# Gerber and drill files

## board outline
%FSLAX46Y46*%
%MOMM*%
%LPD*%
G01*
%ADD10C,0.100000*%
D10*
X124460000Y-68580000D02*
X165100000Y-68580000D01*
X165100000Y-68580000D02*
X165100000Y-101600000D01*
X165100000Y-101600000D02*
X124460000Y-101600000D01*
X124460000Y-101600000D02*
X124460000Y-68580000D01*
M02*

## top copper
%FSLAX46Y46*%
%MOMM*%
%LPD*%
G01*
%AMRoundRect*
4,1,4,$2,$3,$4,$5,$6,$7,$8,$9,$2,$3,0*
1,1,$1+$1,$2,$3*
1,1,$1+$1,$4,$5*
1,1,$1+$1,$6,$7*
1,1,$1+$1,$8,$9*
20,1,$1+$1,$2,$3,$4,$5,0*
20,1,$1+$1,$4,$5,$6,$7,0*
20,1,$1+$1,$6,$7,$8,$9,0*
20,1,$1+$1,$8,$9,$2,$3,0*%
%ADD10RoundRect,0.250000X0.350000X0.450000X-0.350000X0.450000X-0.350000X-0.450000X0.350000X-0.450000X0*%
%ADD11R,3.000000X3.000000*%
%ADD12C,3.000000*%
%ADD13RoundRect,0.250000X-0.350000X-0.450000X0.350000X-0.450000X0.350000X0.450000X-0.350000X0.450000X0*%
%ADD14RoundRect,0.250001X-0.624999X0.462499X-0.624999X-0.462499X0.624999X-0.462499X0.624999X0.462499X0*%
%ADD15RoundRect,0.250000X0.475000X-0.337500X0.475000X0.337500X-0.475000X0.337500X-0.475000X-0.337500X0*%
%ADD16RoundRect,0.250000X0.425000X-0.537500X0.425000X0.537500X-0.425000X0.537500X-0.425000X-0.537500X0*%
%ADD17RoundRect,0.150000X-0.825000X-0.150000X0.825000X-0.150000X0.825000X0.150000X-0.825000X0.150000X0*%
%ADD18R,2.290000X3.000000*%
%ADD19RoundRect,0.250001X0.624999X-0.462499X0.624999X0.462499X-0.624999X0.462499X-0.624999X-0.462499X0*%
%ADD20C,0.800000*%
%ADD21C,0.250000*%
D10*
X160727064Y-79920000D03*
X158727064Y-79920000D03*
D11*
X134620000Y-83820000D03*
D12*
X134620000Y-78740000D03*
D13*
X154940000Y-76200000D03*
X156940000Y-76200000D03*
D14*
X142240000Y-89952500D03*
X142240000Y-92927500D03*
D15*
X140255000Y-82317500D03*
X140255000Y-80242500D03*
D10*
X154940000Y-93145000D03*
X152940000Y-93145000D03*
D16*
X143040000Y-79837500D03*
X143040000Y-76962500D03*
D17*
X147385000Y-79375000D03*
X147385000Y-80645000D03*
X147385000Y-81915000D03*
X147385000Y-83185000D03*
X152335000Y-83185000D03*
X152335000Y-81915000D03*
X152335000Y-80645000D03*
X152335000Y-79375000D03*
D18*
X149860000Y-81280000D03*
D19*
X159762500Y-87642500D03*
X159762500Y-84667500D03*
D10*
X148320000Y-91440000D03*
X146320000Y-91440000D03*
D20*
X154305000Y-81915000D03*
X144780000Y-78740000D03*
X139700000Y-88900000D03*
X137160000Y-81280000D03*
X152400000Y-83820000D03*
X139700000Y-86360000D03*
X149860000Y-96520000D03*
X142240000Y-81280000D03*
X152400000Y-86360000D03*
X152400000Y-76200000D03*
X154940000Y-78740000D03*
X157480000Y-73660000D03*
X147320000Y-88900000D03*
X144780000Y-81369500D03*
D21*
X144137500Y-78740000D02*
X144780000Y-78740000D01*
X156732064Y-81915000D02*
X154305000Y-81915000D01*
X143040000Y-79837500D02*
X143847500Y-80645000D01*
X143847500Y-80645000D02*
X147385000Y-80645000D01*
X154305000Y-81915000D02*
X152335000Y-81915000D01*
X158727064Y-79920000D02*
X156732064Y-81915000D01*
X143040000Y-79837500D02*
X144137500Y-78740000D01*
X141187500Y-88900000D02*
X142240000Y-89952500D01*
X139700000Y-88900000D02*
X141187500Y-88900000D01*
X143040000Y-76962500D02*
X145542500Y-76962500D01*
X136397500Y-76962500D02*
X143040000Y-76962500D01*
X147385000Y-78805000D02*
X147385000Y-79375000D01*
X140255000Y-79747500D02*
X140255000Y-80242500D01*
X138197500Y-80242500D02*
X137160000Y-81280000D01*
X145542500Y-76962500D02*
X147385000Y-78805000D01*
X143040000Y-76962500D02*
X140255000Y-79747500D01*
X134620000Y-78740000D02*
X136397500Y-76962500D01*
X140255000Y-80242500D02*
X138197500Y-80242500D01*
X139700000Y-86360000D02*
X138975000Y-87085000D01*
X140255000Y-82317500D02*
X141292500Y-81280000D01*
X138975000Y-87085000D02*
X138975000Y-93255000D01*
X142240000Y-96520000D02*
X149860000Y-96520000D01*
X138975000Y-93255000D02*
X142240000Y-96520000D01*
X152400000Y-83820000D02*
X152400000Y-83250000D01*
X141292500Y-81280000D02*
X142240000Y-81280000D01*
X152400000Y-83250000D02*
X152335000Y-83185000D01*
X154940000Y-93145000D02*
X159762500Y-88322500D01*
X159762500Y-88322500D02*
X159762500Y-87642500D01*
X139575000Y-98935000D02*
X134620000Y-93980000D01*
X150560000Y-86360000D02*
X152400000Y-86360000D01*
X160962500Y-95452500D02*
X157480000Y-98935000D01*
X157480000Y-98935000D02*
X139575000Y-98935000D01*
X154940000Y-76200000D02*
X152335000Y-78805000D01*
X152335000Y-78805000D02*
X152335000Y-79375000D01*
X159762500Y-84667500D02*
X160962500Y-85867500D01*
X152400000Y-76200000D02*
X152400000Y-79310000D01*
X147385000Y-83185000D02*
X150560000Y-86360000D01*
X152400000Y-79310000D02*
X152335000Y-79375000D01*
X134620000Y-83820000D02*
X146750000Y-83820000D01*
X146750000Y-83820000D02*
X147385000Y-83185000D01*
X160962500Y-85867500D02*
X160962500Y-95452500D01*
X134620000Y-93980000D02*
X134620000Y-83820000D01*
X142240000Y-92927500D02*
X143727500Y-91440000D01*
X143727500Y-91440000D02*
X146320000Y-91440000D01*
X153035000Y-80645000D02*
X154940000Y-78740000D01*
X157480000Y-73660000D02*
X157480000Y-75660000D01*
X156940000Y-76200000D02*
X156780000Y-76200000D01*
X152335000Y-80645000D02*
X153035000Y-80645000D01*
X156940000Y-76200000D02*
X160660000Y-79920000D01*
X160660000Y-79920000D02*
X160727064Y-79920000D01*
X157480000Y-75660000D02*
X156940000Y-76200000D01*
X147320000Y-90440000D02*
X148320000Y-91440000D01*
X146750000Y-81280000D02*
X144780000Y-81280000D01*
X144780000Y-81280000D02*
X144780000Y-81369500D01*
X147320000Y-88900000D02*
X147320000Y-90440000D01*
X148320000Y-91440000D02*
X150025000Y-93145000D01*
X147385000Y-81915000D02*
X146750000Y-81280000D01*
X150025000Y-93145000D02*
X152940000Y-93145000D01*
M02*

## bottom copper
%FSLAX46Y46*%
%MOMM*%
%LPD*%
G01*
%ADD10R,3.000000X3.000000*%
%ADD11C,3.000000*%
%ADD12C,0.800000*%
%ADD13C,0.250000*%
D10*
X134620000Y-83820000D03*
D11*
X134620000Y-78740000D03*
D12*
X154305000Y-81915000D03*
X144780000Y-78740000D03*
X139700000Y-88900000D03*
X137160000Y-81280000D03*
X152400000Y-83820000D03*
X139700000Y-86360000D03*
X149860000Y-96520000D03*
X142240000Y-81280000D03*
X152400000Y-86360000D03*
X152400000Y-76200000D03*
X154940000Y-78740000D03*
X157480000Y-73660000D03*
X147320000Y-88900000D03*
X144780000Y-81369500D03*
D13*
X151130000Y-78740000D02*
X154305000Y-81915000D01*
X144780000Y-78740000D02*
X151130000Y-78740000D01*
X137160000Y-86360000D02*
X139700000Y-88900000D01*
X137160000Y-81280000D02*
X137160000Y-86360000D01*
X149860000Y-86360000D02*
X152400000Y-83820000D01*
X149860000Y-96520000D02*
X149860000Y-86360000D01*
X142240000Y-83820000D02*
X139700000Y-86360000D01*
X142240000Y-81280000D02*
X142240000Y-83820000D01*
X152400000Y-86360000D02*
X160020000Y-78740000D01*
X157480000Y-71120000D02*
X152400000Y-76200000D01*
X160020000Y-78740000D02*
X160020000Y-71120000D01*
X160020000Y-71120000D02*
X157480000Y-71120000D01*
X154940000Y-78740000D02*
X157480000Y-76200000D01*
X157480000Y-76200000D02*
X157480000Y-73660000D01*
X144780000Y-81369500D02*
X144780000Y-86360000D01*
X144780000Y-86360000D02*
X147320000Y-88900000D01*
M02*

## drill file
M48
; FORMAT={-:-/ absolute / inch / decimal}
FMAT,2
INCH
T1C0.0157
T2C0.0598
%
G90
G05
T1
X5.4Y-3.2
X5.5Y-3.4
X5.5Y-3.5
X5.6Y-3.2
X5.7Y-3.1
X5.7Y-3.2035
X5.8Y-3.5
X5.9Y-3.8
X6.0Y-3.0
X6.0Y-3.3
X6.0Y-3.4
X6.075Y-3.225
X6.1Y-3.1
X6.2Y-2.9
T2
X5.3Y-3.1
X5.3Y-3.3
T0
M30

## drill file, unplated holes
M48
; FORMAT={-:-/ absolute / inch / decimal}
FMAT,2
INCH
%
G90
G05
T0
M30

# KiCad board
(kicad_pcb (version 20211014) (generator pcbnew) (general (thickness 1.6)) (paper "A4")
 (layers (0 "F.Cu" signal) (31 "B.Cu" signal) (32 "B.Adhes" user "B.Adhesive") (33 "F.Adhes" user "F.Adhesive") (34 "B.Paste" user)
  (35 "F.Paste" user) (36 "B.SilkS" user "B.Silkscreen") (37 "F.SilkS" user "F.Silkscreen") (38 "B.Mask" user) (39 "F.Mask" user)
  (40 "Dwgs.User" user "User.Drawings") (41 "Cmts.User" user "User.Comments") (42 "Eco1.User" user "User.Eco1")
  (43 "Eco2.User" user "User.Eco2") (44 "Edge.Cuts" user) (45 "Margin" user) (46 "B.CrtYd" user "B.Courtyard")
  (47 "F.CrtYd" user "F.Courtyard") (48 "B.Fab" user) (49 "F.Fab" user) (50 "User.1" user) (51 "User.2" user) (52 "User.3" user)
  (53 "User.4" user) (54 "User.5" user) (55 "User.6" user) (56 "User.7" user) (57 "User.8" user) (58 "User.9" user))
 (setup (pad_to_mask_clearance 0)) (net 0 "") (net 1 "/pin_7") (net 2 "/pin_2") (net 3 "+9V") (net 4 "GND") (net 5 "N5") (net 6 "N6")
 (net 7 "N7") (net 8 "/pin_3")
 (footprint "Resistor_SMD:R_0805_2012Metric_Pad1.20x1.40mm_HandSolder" (layer "F.Cu") (at 159.727064 79.92 180)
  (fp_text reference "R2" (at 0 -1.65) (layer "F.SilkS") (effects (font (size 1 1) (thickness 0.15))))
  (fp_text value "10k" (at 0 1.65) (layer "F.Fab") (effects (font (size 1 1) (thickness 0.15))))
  (pad "1" smd roundrect (at -1 0 180) (size 1.2 1.4) (layers "F.Cu" "F.Paste" "F.Mask") (roundrect_rratio 0.2083333333) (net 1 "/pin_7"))
  (pad "2" smd roundrect (at 1 0 180) (size 1.2 1.4) (layers "F.Cu" "F.Paste" "F.Mask") (roundrect_rratio 0.2083333333) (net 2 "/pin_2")))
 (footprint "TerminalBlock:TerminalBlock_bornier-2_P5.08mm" (layer "F.Cu") (at 134.62 83.82 90)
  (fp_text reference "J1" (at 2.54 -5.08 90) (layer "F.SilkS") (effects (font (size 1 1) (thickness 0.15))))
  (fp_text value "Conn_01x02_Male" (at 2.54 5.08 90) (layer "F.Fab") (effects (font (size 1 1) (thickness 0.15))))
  (pad "1" thru_hole rect (at 0 0 90) (size 3 3) (drill 1.52) (layers *.Cu *.Mask) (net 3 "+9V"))
  (pad "2" thru_hole circle (at 5.08 0 90) (size 3 3) (drill 1.52) (layers *.Cu *.Mask) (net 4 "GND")))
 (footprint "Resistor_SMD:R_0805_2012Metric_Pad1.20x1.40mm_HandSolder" (layer "F.Cu") (at 155.94 76.2)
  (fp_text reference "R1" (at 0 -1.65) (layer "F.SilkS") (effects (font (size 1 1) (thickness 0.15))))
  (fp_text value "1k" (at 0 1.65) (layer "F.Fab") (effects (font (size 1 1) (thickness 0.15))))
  (pad "1" smd roundrect (at -1 0) (size 1.2 1.4) (layers "F.Cu" "F.Paste" "F.Mask") (roundrect_rratio 0.2083333333) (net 3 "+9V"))
  (pad "2" smd roundrect (at 1 0) (size 1.2 1.4) (layers "F.Cu" "F.Paste" "F.Mask") (roundrect_rratio 0.2083333333) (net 1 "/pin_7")))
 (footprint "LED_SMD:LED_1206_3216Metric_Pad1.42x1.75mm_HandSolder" (layer "F.Cu") (at 142.24 91.44 -90)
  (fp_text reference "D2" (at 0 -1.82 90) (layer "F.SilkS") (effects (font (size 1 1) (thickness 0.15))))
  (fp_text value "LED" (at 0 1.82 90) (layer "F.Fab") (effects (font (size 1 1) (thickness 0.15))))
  (pad "1" smd roundrect (at -1.4875 0 270) (size 1.425 1.75) (layers "F.Cu" "F.Paste" "F.Mask") (roundrect_rratio 0.1754392982)
   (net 4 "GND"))
  (pad "2" smd roundrect (at 1.4875 0 270) (size 1.425 1.75) (layers "F.Cu" "F.Paste" "F.Mask") (roundrect_rratio 0.1754392982) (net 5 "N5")))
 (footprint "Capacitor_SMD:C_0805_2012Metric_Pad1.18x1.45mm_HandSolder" (layer "F.Cu") (at 140.255 81.28 90)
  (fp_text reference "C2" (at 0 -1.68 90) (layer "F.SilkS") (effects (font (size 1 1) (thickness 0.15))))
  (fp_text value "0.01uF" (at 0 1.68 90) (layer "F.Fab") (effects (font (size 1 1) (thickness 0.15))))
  (pad "1" smd roundrect (at -1.0375 0 90) (size 1.175 1.45) (layers "F.Cu" "F.Paste" "F.Mask") (roundrect_rratio 0.2127659574) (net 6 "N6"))
  (pad "2" smd roundrect (at 1.0375 0 90) (size 1.175 1.45) (layers "F.Cu" "F.Paste" "F.Mask") (roundrect_rratio 0.2127659574) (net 4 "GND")))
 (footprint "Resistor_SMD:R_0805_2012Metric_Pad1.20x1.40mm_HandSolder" (layer "F.Cu") (at 153.94 93.145 180)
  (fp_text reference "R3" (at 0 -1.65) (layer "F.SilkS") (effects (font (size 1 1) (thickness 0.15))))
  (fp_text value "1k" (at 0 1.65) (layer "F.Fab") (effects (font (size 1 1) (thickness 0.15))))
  (pad "1" smd roundrect (at -1 0 180) (size 1.2 1.4) (layers "F.Cu" "F.Paste" "F.Mask") (roundrect_rratio 0.2083333333) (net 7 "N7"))
  (pad "2" smd roundrect (at 1 0 180) (size 1.2 1.4) (layers "F.Cu" "F.Paste" "F.Mask") (roundrect_rratio 0.2083333333) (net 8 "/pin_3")))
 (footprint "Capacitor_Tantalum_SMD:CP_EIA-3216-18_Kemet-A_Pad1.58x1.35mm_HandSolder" (layer "F.Cu") (at 143.04 78.4 90)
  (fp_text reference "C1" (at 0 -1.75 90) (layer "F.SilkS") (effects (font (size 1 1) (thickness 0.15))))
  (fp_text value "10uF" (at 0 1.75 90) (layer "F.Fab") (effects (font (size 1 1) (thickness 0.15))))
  (pad "1" smd roundrect (at -1.4375 0 90) (size 1.575 1.35) (layers "F.Cu" "F.Paste" "F.Mask") (roundrect_rratio 0.1851851852)
   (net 2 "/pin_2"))
  (pad "2" smd roundrect (at 1.4375 0 90) (size 1.575 1.35) (layers "F.Cu" "F.Paste" "F.Mask") (roundrect_rratio 0.1851851852) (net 4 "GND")))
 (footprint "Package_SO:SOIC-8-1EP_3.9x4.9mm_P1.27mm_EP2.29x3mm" (layer "F.Cu") (at 149.86 81.28)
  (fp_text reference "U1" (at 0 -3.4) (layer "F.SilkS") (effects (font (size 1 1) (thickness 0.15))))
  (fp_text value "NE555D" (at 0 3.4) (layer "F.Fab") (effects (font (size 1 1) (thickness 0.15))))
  (pad "" smd roundrect (at 0.57 0.75) (size 0.92 1.21) (layers "F.Paste") (roundrect_rratio 0.25))
  (pad "" smd roundrect (at -0.57 -0.75) (size 0.92 1.21) (layers "F.Paste") (roundrect_rratio 0.25))
  (pad "" smd roundrect (at -0.57 0.75) (size 0.92 1.21) (layers "F.Paste") (roundrect_rratio 0.25))
  (pad "" smd roundrect (at 0.57 -0.75) (size 0.92 1.21) (layers "F.Paste") (roundrect_rratio 0.25))
  (pad "1" smd roundrect (at -2.475 -1.905) (size 1.95 0.6) (layers "F.Cu" "F.Paste" "F.Mask") (roundrect_rratio 0.25) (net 4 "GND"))
  (pad "2" smd roundrect (at -2.475 -0.635) (size 1.95 0.6) (layers "F.Cu" "F.Paste" "F.Mask") (roundrect_rratio 0.25) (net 2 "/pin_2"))
  (pad "3" smd roundrect (at -2.475 0.635) (size 1.95 0.6) (layers "F.Cu" "F.Paste" "F.Mask") (roundrect_rratio 0.25) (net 8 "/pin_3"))
  (pad "4" smd roundrect (at -2.475 1.905) (size 1.95 0.6) (layers "F.Cu" "F.Paste" "F.Mask") (roundrect_rratio 0.25) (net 3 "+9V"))
  (pad "5" smd roundrect (at 2.475 1.905) (size 1.95 0.6) (layers "F.Cu" "F.Paste" "F.Mask") (roundrect_rratio 0.25) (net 6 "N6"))
  (pad "6" smd roundrect (at 2.475 0.635) (size 1.95 0.6) (layers "F.Cu" "F.Paste" "F.Mask") (roundrect_rratio 0.25) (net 2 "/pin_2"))
  (pad "7" smd roundrect (at 2.475 -0.635) (size 1.95 0.6) (layers "F.Cu" "F.Paste" "F.Mask") (roundrect_rratio 0.25) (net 1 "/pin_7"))
  (pad "8" smd roundrect (at 2.475 -1.905) (size 1.95 0.6) (layers "F.Cu" "F.Paste" "F.Mask") (roundrect_rratio 0.25) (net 3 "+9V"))
  (pad "9" smd rect (at 0 0) (size 2.29 3) (layers "F.Cu" "F.Mask")))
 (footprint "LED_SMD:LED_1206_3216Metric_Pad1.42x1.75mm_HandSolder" (layer "F.Cu") (at 159.7625 86.155 90)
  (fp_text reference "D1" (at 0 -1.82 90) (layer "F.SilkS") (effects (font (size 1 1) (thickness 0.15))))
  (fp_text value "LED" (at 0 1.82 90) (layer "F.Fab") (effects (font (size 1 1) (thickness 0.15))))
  (pad "1" smd roundrect (at -1.4875 0 90) (size 1.425 1.75) (layers "F.Cu" "F.Paste" "F.Mask") (roundrect_rratio 0.1754392982) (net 7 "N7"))
  (pad "2" smd roundrect (at 1.4875 0 90) (size 1.425 1.75) (layers "F.Cu" "F.Paste" "F.Mask") (roundrect_rratio 0.1754392982) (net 3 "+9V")))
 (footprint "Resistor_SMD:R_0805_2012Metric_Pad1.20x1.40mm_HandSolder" (layer "F.Cu") (at 147.32 91.44 180)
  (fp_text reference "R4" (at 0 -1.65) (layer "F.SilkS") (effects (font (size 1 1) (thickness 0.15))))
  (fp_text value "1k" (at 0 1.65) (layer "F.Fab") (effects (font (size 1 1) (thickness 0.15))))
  (pad "1" smd roundrect (at -1 0 180) (size 1.2 1.4) (layers "F.Cu" "F.Paste" "F.Mask") (roundrect_rratio 0.2083333333) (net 8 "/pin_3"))
  (pad "2" smd roundrect (at 1 0 180) (size 1.2 1.4) (layers "F.Cu" "F.Paste" "F.Mask") (roundrect_rratio 0.2083333333) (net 5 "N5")))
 (gr_rect (start 124.46 68.58) (end 165.1 101.6) (layer "Edge.Cuts") (width 0.1) (fill none))
 (segment (start 144.1375 78.74) (end 144.78 78.74) (width 0.25) (layer "F.Cu") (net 2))
 (segment (start 156.732064 81.915) (end 154.305 81.915) (width 0.25) (layer "F.Cu") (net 2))
 (segment (start 143.04 79.8375) (end 143.8475 80.645) (width 0.25) (layer "F.Cu") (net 2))
 (segment (start 143.8475 80.645) (end 147.385 80.645) (width 0.25) (layer "F.Cu") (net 2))
 (segment (start 154.305 81.915) (end 152.335 81.915) (width 0.25) (layer "F.Cu") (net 2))
 (segment (start 158.727064 79.92) (end 156.732064 81.915) (width 0.25) (layer "F.Cu") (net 2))
 (segment (start 143.04 79.8375) (end 144.1375 78.74) (width 0.25) (layer "F.Cu") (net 2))
 (via (at 154.305 81.915) (size 0.8) (drill 0.4) (layers "F.Cu" "B.Cu") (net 2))
 (via (at 144.78 78.74) (size 0.8) (drill 0.4) (layers "F.Cu" "B.Cu") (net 2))
 (segment (start 151.13 78.74) (end 154.305 81.915) (width 0.25) (layer "B.Cu") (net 2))
 (segment (start 144.78 78.74) (end 151.13 78.74) (width 0.25) (layer "B.Cu") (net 2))
 (segment (start 141.1875 88.9) (end 142.24 89.9525) (width 0.25) (layer "F.Cu") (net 4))
 (segment (start 139.7 88.9) (end 141.1875 88.9) (width 0.25) (layer "F.Cu") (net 4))
 (segment (start 143.04 76.9625) (end 145.5425 76.9625) (width 0.25) (layer "F.Cu") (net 4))
 (segment (start 136.3975 76.9625) (end 143.04 76.9625) (width 0.25) (layer "F.Cu") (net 4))
 (segment (start 147.385 78.805) (end 147.385 79.375) (width 0.25) (layer "F.Cu") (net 4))
 (segment (start 140.255 79.7475) (end 140.255 80.2425) (width 0.25) (layer "F.Cu") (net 4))
 (segment (start 138.1975 80.2425) (end 137.16 81.28) (width 0.25) (layer "F.Cu") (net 4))
 (segment (start 145.5425 76.9625) (end 147.385 78.805) (width 0.25) (layer "F.Cu") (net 4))
 (segment (start 143.04 76.9625) (end 140.255 79.7475) (width 0.25) (layer "F.Cu") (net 4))
 (segment (start 134.62 78.74) (end 136.3975 76.9625) (width 0.25) (layer "F.Cu") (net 4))
 (segment (start 140.255 80.2425) (end 138.1975 80.2425) (width 0.25) (layer "F.Cu") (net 4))
 (via (at 139.7 88.9) (size 0.8) (drill 0.4) (layers "F.Cu" "B.Cu") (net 4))
 (via (at 137.16 81.28) (size 0.8) (drill 0.4) (layers "F.Cu" "B.Cu") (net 4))
 (segment (start 137.16 86.36) (end 139.7 88.9) (width 0.25) (layer "B.Cu") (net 4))
 (segment (start 137.16 81.28) (end 137.16 86.36) (width 0.25) (layer "B.Cu") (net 4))
 (segment (start 139.7 86.36) (end 138.975 87.085) (width 0.25) (layer "F.Cu") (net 6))
 (segment (start 140.255 82.3175) (end 141.2925 81.28) (width 0.25) (layer "F.Cu") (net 6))
 (segment (start 138.975 87.085) (end 138.975 93.255) (width 0.25) (layer "F.Cu") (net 6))
 (segment (start 142.24 96.52) (end 149.86 96.52) (width 0.25) (layer "F.Cu") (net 6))
 (segment (start 138.975 93.255) (end 142.24 96.52) (width 0.25) (layer "F.Cu") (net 6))
 (segment (start 152.4 83.82) (end 152.4 83.25) (width 0.25) (layer "F.Cu") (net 6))
 (segment (start 141.2925 81.28) (end 142.24 81.28) (width 0.25) (layer "F.Cu") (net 6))
 (segment (start 152.4 83.25) (end 152.335 83.185) (width 0.25) (layer "F.Cu") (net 6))
 (via (at 152.4 83.82) (size 0.8) (drill 0.4) (layers "F.Cu" "B.Cu") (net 6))
 (via (at 139.7 86.36) (size 0.8) (drill 0.4) (layers "F.Cu" "B.Cu") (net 6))
 (via (at 149.86 96.52) (size 0.8) (drill 0.4) (layers "F.Cu" "B.Cu") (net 6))
 (via (at 142.24 81.28) (size 0.8) (drill 0.4) (layers "F.Cu" "B.Cu") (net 6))
 (segment (start 149.86 86.36) (end 152.4 83.82) (width 0.25) (layer "B.Cu") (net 6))
 (segment (start 149.86 96.52) (end 149.86 86.36) (width 0.25) (layer "B.Cu") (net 6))
 (segment (start 142.24 83.82) (end 139.7 86.36) (width 0.25) (layer "B.Cu") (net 6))
 (segment (start 142.24 81.28) (end 142.24 83.82) (width 0.25) (layer "B.Cu") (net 6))
 (segment (start 154.94 93.145) (end 159.7625 88.3225) (width 0.25) (layer "F.Cu") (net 7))
 (segment (start 159.7625 88.3225) (end 159.7625 87.6425) (width 0.25) (layer "F.Cu") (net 7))
 (segment (start 139.575 98.935) (end 134.62 93.98) (width 0.25) (layer "F.Cu") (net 3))
 (segment (start 150.56 86.36) (end 152.4 86.36) (width 0.25) (layer "F.Cu") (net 3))
 (segment (start 160.9625 95.4525) (end 157.48 98.935) (width 0.25) (layer "F.Cu") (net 3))
 (segment (start 157.48 98.935) (end 139.575 98.935) (width 0.25) (layer "F.Cu") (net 3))
 (segment (start 154.94 76.2) (end 152.335 78.805) (width 0.25) (layer "F.Cu") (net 3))
 (segment (start 152.335 78.805) (end 152.335 79.375) (width 0.25) (layer "F.Cu") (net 3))
 (segment (start 159.7625 84.6675) (end 160.9625 85.8675) (width 0.25) (layer "F.Cu") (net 3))
 (segment (start 152.4 76.2) (end 152.4 79.31) (width 0.25) (layer "F.Cu") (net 3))
 (segment (start 147.385 83.185) (end 150.56 86.36) (width 0.25) (layer "F.Cu") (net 3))
 (segment (start 152.4 79.31) (end 152.335 79.375) (width 0.25) (layer "F.Cu") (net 3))
 (segment (start 134.62 83.82) (end 146.75 83.82) (width 0.25) (layer "F.Cu") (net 3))
 (segment (start 146.75 83.82) (end 147.385 83.185) (width 0.25) (layer "F.Cu") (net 3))
 (segment (start 160.9625 85.8675) (end 160.9625 95.4525) (width 0.25) (layer "F.Cu") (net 3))
 (segment (start 134.62 93.98) (end 134.62 83.82) (width 0.25) (layer "F.Cu") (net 3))
 (via (at 152.4 86.36) (size 0.8) (drill 0.4) (layers "F.Cu" "B.Cu") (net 3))
 (via (at 152.4 76.2) (size 0.8) (drill 0.4) (layers "F.Cu" "B.Cu") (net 3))
 (segment (start 152.4 86.36) (end 160.02 78.74) (width 0.25) (layer "B.Cu") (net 3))
 (segment (start 157.48 71.12) (end 152.4 76.2) (width 0.25) (layer "B.Cu") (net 3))
 (segment (start 160.02 78.74) (end 160.02 71.12) (width 0.25) (layer "B.Cu") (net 3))
 (segment (start 160.02 71.12) (end 157.48 71.12) (width 0.25) (layer "B.Cu") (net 3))
 (segment (start 142.24 92.9275) (end 143.7275 91.44) (width 0.25) (layer "F.Cu") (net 5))
 (segment (start 143.7275 91.44) (end 146.32 91.44) (width 0.25) (layer "F.Cu") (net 5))
 (segment (start 153.035 80.645) (end 154.94 78.74) (width 0.25) (layer "F.Cu") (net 1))
 (segment (start 157.48 73.66) (end 157.48 75.66) (width 0.25) (layer "F.Cu") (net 1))
 (segment (start 156.94 76.2) (end 156.78 76.2) (width 0.25) (layer "F.Cu") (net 1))
 (segment (start 152.335 80.645) (end 153.035 80.645) (width 0.25) (layer "F.Cu") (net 1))
 (segment (start 156.94 76.2) (end 160.66 79.92) (width 0.25) (layer "F.Cu") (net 1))
 (segment (start 160.66 79.92) (end 160.727064 79.92) (width 0.25) (layer "F.Cu") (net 1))
 (segment (start 157.48 75.66) (end 156.94 76.2) (width 0.25) (layer "F.Cu") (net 1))
 (via (at 154.94 78.74) (size 0.8) (drill 0.4) (layers "F.Cu" "B.Cu") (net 1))
 (via (at 157.48 73.66) (size 0.8) (drill 0.4) (layers "F.Cu" "B.Cu") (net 1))
 (segment (start 154.94 78.74) (end 157.48 76.2) (width 0.25) (layer "B.Cu") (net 1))
 (segment (start 157.48 76.2) (end 157.48 73.66) (width 0.25) (layer "B.Cu") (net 1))
 (segment (start 147.32 90.44) (end 148.32 91.44) (width 0.25) (layer "F.Cu") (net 8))
 (segment (start 146.75 81.28) (end 144.78 81.28) (width 0.25) (layer "F.Cu") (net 8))
 (segment (start 144.78 81.28) (end 144.78 81.3695) (width 0.25) (layer "F.Cu") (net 8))
 (segment (start 147.32 88.9) (end 147.32 90.44) (width 0.25) (layer "F.Cu") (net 8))
 (segment (start 148.32 91.44) (end 150.025 93.145) (width 0.25) (layer "F.Cu") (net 8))
 (segment (start 147.385 81.915) (end 146.75 81.28) (width 0.25) (layer "F.Cu") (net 8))
 (segment (start 150.025 93.145) (end 152.94 93.145) (width 0.25) (layer "F.Cu") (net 8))
 (via (at 147.32 88.9) (size 0.8) (drill 0.4) (layers "F.Cu" "B.Cu") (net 8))
 (via (at 144.78 81.3695) (size 0.8) (drill 0.4) (layers "F.Cu" "B.Cu") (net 8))
 (segment (start 144.78 81.3695) (end 144.78 86.36) (width 0.25) (layer "B.Cu") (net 8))
 (segment (start 144.78 86.36) (end 147.32 88.9) (width 0.25) (layer "B.Cu") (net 8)))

